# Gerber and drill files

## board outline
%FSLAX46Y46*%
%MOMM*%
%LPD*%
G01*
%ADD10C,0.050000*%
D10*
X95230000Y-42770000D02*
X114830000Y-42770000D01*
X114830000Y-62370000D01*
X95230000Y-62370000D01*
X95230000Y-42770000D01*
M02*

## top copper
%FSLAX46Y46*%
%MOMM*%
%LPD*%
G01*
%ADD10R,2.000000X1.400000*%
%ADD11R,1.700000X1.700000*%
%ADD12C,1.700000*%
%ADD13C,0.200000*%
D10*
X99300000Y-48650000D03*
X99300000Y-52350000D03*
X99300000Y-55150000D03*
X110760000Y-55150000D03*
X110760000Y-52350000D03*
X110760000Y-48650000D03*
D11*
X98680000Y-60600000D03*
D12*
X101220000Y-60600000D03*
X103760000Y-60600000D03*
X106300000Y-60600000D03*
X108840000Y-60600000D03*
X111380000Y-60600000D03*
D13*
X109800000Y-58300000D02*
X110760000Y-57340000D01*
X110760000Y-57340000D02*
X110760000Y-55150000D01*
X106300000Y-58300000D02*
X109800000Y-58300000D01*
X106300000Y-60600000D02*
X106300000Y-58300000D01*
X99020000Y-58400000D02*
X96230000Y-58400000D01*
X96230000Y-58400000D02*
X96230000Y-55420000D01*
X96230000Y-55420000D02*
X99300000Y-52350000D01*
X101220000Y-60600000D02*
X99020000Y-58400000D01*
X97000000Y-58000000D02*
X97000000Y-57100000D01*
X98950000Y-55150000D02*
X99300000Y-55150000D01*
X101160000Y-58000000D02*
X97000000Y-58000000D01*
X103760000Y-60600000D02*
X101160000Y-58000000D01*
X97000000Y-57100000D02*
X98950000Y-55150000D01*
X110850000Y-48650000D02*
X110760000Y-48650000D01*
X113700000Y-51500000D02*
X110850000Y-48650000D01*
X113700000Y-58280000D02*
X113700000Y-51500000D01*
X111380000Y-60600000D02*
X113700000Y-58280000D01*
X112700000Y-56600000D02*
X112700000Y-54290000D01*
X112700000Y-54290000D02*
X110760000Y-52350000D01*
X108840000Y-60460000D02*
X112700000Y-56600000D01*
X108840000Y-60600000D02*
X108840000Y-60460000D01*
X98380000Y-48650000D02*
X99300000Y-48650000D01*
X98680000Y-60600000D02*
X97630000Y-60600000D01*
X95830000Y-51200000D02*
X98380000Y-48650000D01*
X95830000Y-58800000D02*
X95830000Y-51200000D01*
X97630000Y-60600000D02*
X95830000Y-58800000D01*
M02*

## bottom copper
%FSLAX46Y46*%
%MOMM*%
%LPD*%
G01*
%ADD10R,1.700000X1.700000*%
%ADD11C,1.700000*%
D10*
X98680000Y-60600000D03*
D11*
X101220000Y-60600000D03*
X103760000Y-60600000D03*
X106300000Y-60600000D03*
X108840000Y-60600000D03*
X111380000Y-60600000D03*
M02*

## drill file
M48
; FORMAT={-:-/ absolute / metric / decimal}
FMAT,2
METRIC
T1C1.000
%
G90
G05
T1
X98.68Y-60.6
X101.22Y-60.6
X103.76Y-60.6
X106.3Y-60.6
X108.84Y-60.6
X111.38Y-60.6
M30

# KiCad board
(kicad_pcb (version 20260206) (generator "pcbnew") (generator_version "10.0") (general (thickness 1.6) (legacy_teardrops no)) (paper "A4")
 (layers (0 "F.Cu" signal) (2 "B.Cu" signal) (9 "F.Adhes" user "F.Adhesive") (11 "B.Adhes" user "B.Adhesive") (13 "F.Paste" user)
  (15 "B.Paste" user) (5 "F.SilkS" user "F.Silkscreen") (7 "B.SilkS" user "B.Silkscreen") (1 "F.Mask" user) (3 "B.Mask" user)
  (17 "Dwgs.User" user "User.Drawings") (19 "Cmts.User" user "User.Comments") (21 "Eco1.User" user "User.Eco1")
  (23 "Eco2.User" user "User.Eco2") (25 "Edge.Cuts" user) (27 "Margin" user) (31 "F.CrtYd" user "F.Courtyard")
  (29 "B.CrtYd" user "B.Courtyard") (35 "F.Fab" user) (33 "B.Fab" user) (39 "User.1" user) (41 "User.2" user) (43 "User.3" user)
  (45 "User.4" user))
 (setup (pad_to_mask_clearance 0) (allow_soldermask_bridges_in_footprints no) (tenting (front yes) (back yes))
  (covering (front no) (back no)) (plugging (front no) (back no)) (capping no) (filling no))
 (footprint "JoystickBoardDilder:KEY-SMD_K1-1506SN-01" (layer "F.Cu") (at 105.03 51.9)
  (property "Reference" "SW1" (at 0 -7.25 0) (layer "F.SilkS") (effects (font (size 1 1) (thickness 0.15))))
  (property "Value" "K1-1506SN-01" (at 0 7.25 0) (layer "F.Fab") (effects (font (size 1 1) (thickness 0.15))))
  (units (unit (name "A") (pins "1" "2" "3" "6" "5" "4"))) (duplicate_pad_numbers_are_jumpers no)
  (pad "1" smd rect (at -5.73 -3.25) (size 2 1.4) (layers "F.Cu" "F.Mask" "F.Paste") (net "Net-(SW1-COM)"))
  (pad "2" smd rect (at -5.73 0.45) (size 2 1.4) (layers "F.Cu" "F.Mask" "F.Paste") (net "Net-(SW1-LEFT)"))
  (pad "3" smd rect (at -5.73 3.25) (size 2 1.4) (layers "F.Cu" "F.Mask" "F.Paste") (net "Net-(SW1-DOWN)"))
  (pad "4" smd rect (at 5.73 3.25) (size 2 1.4) (layers "F.Cu" "F.Mask" "F.Paste") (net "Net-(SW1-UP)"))
  (pad "5" smd rect (at 5.73 0.45) (size 2 1.4) (layers "F.Cu" "F.Mask" "F.Paste") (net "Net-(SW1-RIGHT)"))
  (pad "6" smd rect (at 5.73 -3.25) (size 2 1.4) (layers "F.Cu" "F.Mask" "F.Paste") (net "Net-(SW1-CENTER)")))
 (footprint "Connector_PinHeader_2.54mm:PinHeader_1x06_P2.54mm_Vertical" (layer "F.Cu") (at 98.68 60.6 90)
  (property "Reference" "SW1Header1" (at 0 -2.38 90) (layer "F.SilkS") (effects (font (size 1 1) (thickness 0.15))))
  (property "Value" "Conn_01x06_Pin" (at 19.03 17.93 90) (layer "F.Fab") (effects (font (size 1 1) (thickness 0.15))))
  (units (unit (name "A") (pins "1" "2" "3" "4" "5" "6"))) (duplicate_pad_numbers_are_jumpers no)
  (pad "1" thru_hole rect (at 0 0 90) (size 1.7 1.7) (drill 1) (layers "*.Cu" "*.Mask") (remove_unused_layers no) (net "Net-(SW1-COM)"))
  (pad "2" thru_hole circle (at 0 2.54 90) (size 1.7 1.7) (drill 1) (layers "*.Cu" "*.Mask") (remove_unused_layers no)
   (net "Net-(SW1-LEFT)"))
  (pad "3" thru_hole circle (at 0 5.08 90) (size 1.7 1.7) (drill 1) (layers "*.Cu" "*.Mask") (remove_unused_layers no)
   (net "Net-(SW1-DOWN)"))
  (pad "4" thru_hole circle (at 0 7.62 90) (size 1.7 1.7) (drill 1) (layers "*.Cu" "*.Mask") (remove_unused_layers no) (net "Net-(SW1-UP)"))
  (pad "5" thru_hole circle (at 0 10.16 90) (size 1.7 1.7) (drill 1) (layers "*.Cu" "*.Mask") (remove_unused_layers no)
   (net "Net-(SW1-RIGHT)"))
  (pad "6" thru_hole circle (at 0 12.7 90) (size 1.7 1.7) (drill 1) (layers "*.Cu" "*.Mask") (remove_unused_layers no)
   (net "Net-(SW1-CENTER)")))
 (gr_rect (start 95.23 42.77) (end 114.83 62.37) (stroke (width 0.05) (type default)) (fill no) (layer "Edge.Cuts"))
 (segment (start 109.8 58.3) (end 110.76 57.34) (width 0.2) (layer "F.Cu") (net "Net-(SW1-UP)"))
 (segment (start 110.76 57.34) (end 110.76 55.15) (width 0.2) (layer "F.Cu") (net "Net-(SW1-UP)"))
 (segment (start 106.3 58.3) (end 109.8 58.3) (width 0.2) (layer "F.Cu") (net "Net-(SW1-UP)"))
 (segment (start 106.3 60.6) (end 106.3 58.3) (width 0.2) (layer "F.Cu") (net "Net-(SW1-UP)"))
 (segment (start 99.02 58.4) (end 96.23 58.4) (width 0.2) (layer "F.Cu") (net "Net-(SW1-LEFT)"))
 (segment (start 96.23 58.4) (end 96.23 55.42) (width 0.2) (layer "F.Cu") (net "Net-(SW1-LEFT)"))
 (segment (start 96.23 55.42) (end 99.3 52.35) (width 0.2) (layer "F.Cu") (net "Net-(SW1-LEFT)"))
 (segment (start 101.22 60.6) (end 99.02 58.4) (width 0.2) (layer "F.Cu") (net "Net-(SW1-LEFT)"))
 (segment (start 97 58) (end 97 57.1) (width 0.2) (layer "F.Cu") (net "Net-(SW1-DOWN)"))
 (segment (start 98.95 55.15) (end 99.3 55.15) (width 0.2) (layer "F.Cu") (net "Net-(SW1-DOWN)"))
 (segment (start 101.16 58) (end 97 58) (width 0.2) (layer "F.Cu") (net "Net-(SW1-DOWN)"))
 (segment (start 103.76 60.6) (end 101.16 58) (width 0.2) (layer "F.Cu") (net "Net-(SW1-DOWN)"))
 (segment (start 97 57.1) (end 98.95 55.15) (width 0.2) (layer "F.Cu") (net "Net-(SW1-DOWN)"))
 (segment (start 110.85 48.65) (end 110.76 48.65) (width 0.2) (layer "F.Cu") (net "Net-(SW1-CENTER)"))
 (segment (start 113.7 51.5) (end 110.85 48.65) (width 0.2) (layer "F.Cu") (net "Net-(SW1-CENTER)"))
 (segment (start 113.7 58.28) (end 113.7 51.5) (width 0.2) (layer "F.Cu") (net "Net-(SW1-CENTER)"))
 (segment (start 111.38 60.6) (end 113.7 58.28) (width 0.2) (layer "F.Cu") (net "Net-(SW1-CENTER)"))
 (segment (start 112.7 56.6) (end 112.7 54.29) (width 0.2) (layer "F.Cu") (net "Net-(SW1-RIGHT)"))
 (segment (start 112.7 54.29) (end 110.76 52.35) (width 0.2) (layer "F.Cu") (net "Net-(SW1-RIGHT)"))
 (segment (start 108.84 60.46) (end 112.7 56.6) (width 0.2) (layer "F.Cu") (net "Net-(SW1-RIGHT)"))
 (segment (start 108.84 60.6) (end 108.84 60.46) (width 0.2) (layer "F.Cu") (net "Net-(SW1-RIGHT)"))
 (segment (start 98.38 48.65) (end 99.3 48.65) (width 0.2) (layer "F.Cu") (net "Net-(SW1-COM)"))
 (segment (start 98.68 60.6) (end 97.63 60.6) (width 0.2) (layer "F.Cu") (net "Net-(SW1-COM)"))
 (segment (start 95.83 51.2) (end 98.38 48.65) (width 0.2) (layer "F.Cu") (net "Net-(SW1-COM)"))
 (segment (start 95.83 58.8) (end 95.83 51.2) (width 0.2) (layer "F.Cu") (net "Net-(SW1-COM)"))
 (segment (start 97.63 60.6) (end 95.83 58.8) (width 0.2) (layer "F.Cu") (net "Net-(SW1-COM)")))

